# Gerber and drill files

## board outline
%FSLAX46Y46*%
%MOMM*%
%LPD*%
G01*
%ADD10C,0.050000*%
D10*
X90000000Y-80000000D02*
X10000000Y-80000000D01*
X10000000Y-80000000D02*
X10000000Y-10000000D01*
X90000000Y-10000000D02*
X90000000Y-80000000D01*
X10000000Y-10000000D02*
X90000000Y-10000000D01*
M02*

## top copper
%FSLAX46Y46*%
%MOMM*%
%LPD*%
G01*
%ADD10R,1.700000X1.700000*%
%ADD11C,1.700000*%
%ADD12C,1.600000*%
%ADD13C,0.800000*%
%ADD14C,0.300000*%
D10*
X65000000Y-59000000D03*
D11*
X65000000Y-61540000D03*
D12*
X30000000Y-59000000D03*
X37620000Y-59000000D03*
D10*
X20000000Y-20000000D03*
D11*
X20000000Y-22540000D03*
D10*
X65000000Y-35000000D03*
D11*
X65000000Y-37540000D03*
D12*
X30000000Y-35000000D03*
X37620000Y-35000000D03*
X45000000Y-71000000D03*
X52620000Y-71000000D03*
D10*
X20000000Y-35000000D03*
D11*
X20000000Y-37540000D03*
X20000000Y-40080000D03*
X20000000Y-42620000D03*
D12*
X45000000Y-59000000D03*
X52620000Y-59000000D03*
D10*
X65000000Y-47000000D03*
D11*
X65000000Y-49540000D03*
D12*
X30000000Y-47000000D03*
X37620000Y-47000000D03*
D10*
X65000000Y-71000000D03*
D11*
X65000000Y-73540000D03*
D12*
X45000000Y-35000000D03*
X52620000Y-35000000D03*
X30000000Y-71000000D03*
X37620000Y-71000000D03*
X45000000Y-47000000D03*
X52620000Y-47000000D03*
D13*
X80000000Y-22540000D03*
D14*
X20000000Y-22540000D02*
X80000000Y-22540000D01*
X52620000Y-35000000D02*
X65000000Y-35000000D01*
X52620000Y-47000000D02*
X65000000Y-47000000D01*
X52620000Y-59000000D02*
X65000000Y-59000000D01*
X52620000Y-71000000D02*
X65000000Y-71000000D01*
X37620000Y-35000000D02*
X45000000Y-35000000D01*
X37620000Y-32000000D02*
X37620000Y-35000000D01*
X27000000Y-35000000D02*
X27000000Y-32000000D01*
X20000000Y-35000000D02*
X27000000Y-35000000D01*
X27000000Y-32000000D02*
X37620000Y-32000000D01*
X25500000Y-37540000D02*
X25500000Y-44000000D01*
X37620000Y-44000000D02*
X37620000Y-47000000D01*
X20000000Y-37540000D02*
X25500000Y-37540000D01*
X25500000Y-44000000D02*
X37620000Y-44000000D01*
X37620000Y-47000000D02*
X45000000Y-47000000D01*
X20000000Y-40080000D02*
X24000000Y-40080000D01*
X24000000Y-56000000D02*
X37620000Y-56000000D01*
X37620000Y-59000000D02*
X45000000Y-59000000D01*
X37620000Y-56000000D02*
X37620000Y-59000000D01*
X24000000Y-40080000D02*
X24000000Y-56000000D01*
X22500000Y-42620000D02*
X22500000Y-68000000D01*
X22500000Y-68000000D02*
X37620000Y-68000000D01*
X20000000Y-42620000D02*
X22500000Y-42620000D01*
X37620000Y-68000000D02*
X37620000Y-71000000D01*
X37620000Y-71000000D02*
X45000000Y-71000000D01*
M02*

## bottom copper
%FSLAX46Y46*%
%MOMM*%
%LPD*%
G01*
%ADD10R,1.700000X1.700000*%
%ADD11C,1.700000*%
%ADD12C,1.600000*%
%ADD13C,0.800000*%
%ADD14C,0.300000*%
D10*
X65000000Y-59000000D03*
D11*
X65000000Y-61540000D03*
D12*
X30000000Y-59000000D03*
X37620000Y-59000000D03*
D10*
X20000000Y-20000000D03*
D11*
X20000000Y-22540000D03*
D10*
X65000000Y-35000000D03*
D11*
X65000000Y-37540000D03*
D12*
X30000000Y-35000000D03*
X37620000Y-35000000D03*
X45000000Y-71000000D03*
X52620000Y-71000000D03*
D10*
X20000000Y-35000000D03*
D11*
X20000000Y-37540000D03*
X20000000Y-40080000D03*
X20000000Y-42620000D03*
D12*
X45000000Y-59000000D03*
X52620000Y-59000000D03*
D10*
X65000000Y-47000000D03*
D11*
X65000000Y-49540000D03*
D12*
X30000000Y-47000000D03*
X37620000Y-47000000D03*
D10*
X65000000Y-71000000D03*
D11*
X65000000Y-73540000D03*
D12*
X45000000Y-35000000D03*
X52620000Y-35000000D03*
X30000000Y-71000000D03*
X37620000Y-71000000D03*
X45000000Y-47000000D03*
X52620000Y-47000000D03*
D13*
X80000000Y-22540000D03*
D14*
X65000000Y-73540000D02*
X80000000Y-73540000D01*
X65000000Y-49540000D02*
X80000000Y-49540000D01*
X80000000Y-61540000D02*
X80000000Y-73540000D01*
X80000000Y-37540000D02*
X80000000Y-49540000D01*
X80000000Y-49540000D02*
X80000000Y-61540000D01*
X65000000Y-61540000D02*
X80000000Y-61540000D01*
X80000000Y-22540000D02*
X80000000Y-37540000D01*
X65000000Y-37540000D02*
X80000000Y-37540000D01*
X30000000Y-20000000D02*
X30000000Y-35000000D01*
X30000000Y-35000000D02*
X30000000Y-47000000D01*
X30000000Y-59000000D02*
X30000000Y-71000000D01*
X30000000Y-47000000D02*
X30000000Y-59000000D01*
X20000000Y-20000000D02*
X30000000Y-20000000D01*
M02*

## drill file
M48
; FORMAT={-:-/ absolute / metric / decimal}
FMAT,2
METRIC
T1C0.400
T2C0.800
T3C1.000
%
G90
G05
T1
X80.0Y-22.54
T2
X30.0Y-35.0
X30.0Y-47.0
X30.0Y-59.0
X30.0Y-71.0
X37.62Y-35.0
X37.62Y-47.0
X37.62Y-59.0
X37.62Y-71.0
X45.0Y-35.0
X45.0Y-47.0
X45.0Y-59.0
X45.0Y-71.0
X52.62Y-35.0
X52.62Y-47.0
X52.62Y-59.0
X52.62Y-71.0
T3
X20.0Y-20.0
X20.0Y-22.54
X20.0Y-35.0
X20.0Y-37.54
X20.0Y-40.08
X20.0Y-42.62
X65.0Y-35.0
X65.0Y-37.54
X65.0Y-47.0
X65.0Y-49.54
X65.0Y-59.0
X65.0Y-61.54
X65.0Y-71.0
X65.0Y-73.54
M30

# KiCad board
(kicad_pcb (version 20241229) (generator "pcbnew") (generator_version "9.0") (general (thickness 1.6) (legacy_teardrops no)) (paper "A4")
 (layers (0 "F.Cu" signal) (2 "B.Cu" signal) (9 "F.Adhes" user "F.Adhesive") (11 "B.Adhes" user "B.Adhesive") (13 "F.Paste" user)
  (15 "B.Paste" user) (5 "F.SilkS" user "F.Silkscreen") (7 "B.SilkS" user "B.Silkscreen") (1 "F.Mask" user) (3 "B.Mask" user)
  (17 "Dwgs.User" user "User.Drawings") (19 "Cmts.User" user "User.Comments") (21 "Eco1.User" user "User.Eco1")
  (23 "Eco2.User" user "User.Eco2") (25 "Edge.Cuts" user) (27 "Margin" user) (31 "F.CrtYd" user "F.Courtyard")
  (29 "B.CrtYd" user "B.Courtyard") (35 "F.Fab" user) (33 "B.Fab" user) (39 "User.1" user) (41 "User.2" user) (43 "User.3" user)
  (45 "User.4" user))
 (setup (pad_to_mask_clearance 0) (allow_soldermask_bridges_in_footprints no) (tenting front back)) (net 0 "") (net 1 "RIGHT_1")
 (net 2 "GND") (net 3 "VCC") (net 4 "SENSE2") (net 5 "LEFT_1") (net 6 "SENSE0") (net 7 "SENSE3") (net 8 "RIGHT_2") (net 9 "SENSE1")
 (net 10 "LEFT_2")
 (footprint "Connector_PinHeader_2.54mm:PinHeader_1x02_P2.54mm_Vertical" (layer "F.Cu") (at 65 59)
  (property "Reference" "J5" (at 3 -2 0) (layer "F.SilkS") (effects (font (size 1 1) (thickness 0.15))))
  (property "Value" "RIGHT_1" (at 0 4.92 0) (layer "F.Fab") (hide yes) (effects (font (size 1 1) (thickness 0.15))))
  (pad "1" thru_hole rect (at 0 0) (size 1.7 1.7) (drill 1) (layers "*.Cu" "*.Mask") (remove_unused_layers no) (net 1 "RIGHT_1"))
  (pad "2" thru_hole circle (at 0 2.54) (size 1.7 1.7) (drill 1) (layers "*.Cu" "*.Mask") (remove_unused_layers no) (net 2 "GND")))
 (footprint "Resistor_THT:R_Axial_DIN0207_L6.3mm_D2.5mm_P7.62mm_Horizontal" (layer "F.Cu") (at 30 59)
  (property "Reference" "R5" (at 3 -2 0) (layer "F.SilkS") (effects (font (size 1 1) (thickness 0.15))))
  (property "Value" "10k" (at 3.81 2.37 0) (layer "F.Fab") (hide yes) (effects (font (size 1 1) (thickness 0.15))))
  (pad "1" thru_hole circle (at 0 0) (size 1.6 1.6) (drill 0.8) (layers "*.Cu" "*.Mask") (remove_unused_layers no) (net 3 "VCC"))
  (pad "2" thru_hole circle (at 7.62 0) (size 1.6 1.6) (drill 0.8) (layers "*.Cu" "*.Mask") (remove_unused_layers no) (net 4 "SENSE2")))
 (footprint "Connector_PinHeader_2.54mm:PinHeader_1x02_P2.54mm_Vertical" (layer "F.Cu") (at 20 20)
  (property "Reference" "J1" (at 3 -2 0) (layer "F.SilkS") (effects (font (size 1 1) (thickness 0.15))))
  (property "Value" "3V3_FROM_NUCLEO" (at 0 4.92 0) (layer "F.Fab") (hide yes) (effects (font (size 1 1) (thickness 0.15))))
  (pad "1" thru_hole rect (at 0 0) (size 1.7 1.7) (drill 1) (layers "*.Cu" "*.Mask") (remove_unused_layers no) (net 3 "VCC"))
  (pad "2" thru_hole circle (at 0 2.54) (size 1.7 1.7) (drill 1) (layers "*.Cu" "*.Mask") (remove_unused_layers no) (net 2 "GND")))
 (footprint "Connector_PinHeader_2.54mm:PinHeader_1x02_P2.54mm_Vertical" (layer "F.Cu") (at 65 35)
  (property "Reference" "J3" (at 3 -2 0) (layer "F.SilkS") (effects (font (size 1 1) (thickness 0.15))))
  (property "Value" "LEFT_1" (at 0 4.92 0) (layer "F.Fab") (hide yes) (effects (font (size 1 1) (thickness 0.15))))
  (pad "1" thru_hole rect (at 0 0) (size 1.7 1.7) (drill 1) (layers "*.Cu" "*.Mask") (remove_unused_layers no) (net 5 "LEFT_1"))
  (pad "2" thru_hole circle (at 0 2.54) (size 1.7 1.7) (drill 1) (layers "*.Cu" "*.Mask") (remove_unused_layers no) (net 2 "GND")))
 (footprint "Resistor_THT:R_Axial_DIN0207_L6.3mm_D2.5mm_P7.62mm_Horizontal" (layer "F.Cu") (at 30 35)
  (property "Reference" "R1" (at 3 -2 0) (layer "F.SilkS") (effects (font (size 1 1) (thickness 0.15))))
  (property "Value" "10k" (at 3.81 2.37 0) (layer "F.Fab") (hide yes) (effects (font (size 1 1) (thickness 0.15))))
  (pad "1" thru_hole circle (at 0 0) (size 1.6 1.6) (drill 0.8) (layers "*.Cu" "*.Mask") (remove_unused_layers no) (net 3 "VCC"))
  (pad "2" thru_hole circle (at 7.62 0) (size 1.6 1.6) (drill 0.8) (layers "*.Cu" "*.Mask") (remove_unused_layers no) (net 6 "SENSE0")))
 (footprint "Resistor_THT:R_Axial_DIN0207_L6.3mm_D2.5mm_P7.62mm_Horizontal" (layer "F.Cu") (at 45 71)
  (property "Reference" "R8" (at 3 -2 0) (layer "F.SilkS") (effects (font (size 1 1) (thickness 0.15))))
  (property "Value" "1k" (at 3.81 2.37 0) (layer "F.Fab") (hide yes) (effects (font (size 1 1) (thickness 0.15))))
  (pad "1" thru_hole circle (at 0 0) (size 1.6 1.6) (drill 0.8) (layers "*.Cu" "*.Mask") (remove_unused_layers no) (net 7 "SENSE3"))
  (pad "2" thru_hole circle (at 7.62 0) (size 1.6 1.6) (drill 0.8) (layers "*.Cu" "*.Mask") (remove_unused_layers no) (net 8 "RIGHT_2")))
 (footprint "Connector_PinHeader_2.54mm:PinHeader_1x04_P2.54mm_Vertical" (layer "F.Cu") (at 20 35)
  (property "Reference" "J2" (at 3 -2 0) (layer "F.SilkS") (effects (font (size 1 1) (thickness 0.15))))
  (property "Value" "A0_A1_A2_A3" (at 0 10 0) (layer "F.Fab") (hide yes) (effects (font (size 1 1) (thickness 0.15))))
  (pad "1" thru_hole rect (at 0 0) (size 1.7 1.7) (drill 1) (layers "*.Cu" "*.Mask") (remove_unused_layers no) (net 6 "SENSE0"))
  (pad "2" thru_hole circle (at 0 2.54) (size 1.7 1.7) (drill 1) (layers "*.Cu" "*.Mask") (remove_unused_layers no) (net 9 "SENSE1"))
  (pad "3" thru_hole circle (at 0 5.08) (size 1.7 1.7) (drill 1) (layers "*.Cu" "*.Mask") (remove_unused_layers no) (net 4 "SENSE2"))
  (pad "4" thru_hole circle (at 0 7.62) (size 1.7 1.7) (drill 1) (layers "*.Cu" "*.Mask") (remove_unused_layers no) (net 7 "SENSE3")))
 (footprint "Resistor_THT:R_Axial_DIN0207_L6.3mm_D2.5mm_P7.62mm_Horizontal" (layer "F.Cu") (at 45 59)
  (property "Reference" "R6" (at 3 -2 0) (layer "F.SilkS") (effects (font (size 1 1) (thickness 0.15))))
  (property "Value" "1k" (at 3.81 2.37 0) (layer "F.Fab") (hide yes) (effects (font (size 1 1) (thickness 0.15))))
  (pad "1" thru_hole circle (at 0 0) (size 1.6 1.6) (drill 0.8) (layers "*.Cu" "*.Mask") (remove_unused_layers no) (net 4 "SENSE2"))
  (pad "2" thru_hole circle (at 7.62 0) (size 1.6 1.6) (drill 0.8) (layers "*.Cu" "*.Mask") (remove_unused_layers no) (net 1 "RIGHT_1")))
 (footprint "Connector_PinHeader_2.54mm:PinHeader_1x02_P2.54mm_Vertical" (layer "F.Cu") (at 65 47)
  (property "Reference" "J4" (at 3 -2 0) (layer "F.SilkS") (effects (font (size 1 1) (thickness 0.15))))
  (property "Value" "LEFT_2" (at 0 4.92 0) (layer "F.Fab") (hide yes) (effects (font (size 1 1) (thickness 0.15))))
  (pad "1" thru_hole rect (at 0 0) (size 1.7 1.7) (drill 1) (layers "*.Cu" "*.Mask") (remove_unused_layers no) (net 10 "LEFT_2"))
  (pad "2" thru_hole circle (at 0 2.54) (size 1.7 1.7) (drill 1) (layers "*.Cu" "*.Mask") (remove_unused_layers no) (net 2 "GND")))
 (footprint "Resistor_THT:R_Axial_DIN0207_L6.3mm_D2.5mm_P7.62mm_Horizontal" (layer "F.Cu") (at 30 47)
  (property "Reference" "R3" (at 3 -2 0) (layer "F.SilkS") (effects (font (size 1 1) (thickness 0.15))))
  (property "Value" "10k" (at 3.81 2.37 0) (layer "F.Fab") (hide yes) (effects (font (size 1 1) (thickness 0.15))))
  (pad "1" thru_hole circle (at 0 0) (size 1.6 1.6) (drill 0.8) (layers "*.Cu" "*.Mask") (remove_unused_layers no) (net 3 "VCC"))
  (pad "2" thru_hole circle (at 7.62 0) (size 1.6 1.6) (drill 0.8) (layers "*.Cu" "*.Mask") (remove_unused_layers no) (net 9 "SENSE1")))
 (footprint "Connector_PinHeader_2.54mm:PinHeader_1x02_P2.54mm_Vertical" (layer "F.Cu") (at 65 71)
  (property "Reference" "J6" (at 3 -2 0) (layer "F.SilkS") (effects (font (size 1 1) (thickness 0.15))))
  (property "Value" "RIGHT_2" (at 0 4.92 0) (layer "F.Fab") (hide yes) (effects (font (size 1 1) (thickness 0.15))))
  (pad "1" thru_hole rect (at 0 0) (size 1.7 1.7) (drill 1) (layers "*.Cu" "*.Mask") (remove_unused_layers no) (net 8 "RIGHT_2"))
  (pad "2" thru_hole circle (at 0 2.54) (size 1.7 1.7) (drill 1) (layers "*.Cu" "*.Mask") (remove_unused_layers no) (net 2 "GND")))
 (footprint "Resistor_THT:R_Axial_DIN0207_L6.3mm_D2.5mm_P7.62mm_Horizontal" (layer "F.Cu") (at 45 35)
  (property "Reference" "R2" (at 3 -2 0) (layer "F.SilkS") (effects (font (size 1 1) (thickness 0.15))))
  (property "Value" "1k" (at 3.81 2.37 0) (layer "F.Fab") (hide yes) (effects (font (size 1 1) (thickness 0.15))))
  (pad "1" thru_hole circle (at 0 0) (size 1.6 1.6) (drill 0.8) (layers "*.Cu" "*.Mask") (remove_unused_layers no) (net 6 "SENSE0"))
  (pad "2" thru_hole circle (at 7.62 0) (size 1.6 1.6) (drill 0.8) (layers "*.Cu" "*.Mask") (remove_unused_layers no) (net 5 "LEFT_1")))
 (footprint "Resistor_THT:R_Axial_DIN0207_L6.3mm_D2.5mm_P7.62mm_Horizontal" (layer "F.Cu") (at 30 71)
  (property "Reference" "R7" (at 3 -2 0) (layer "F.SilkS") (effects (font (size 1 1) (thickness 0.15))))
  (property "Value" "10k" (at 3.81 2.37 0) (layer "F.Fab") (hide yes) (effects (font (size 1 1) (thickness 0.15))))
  (pad "1" thru_hole circle (at 0 0) (size 1.6 1.6) (drill 0.8) (layers "*.Cu" "*.Mask") (remove_unused_layers no) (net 3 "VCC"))
  (pad "2" thru_hole circle (at 7.62 0) (size 1.6 1.6) (drill 0.8) (layers "*.Cu" "*.Mask") (remove_unused_layers no) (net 7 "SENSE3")))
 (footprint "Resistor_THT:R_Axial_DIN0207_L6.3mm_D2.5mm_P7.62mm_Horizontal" (layer "F.Cu") (at 45 47)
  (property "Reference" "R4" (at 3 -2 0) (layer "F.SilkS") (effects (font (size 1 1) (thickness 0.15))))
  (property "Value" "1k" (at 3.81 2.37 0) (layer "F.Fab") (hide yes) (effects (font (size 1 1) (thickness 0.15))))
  (pad "1" thru_hole circle (at 0 0) (size 1.6 1.6) (drill 0.8) (layers "*.Cu" "*.Mask") (remove_unused_layers no) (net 9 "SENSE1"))
  (pad "2" thru_hole circle (at 7.62 0) (size 1.6 1.6) (drill 0.8) (layers "*.Cu" "*.Mask") (remove_unused_layers no) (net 10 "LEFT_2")))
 (gr_line (start 90 80) (end 10 80) (stroke (width 0.05) (type default)) (layer "Edge.Cuts"))
 (gr_line (start 10 80) (end 10 10) (stroke (width 0.05) (type default)) (layer "Edge.Cuts"))
 (gr_line (start 90 10) (end 90 80) (stroke (width 0.05) (type default)) (layer "Edge.Cuts"))
 (gr_line (start 10 10) (end 90 10) (stroke (width 0.05) (type default)) (layer "Edge.Cuts"))
 (segment (start 20 22.54) (end 80 22.54) (width 0.3) (layer "F.Cu") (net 2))
 (via (at 80 22.54) (size 0.8) (drill 0.4) (layers "F.Cu" "B.Cu") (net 2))
 (segment (start 65 73.54) (end 80 73.54) (width 0.3) (layer "B.Cu") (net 2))
 (segment (start 65 49.54) (end 80 49.54) (width 0.3) (layer "B.Cu") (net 2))
 (segment (start 80 61.54) (end 80 73.54) (width 0.3) (layer "B.Cu") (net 2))
 (segment (start 80 37.54) (end 80 49.54) (width 0.3) (layer "B.Cu") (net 2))
 (segment (start 80 49.54) (end 80 61.54) (width 0.3) (layer "B.Cu") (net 2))
 (segment (start 65 61.54) (end 80 61.54) (width 0.3) (layer "B.Cu") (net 2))
 (segment (start 80 22.54) (end 80 37.54) (width 0.3) (layer "B.Cu") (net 2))
 (segment (start 65 37.54) (end 80 37.54) (width 0.3) (layer "B.Cu") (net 2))
 (segment (start 52.62 35) (end 65 35) (width 0.3) (layer "F.Cu") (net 5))
 (segment (start 52.62 47) (end 65 47) (width 0.3) (layer "F.Cu") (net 10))
 (segment (start 52.62 59) (end 65 59) (width 0.3) (layer "F.Cu") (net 1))
 (segment (start 52.62 71) (end 65 71) (width 0.3) (layer "F.Cu") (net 8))
 (segment (start 37.62 35) (end 45 35) (width 0.3) (layer "F.Cu") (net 6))
 (segment (start 37.62 32) (end 37.62 35) (width 0.3) (layer "F.Cu") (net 6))
 (segment (start 27 35) (end 27 32) (width 0.3) (layer "F.Cu") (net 6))
 (segment (start 20 35) (end 27 35) (width 0.3) (layer "F.Cu") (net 6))
 (segment (start 27 32) (end 37.62 32) (width 0.3) (layer "F.Cu") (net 6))
 (segment (start 25.5 37.54) (end 25.5 44) (width 0.3) (layer "F.Cu") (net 9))
 (segment (start 37.62 44) (end 37.62 47) (width 0.3) (layer "F.Cu") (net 9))
 (segment (start 20 37.54) (end 25.5 37.54) (width 0.3) (layer "F.Cu") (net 9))
 (segment (start 25.5 44) (end 37.62 44) (width 0.3) (layer "F.Cu") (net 9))
 (segment (start 37.62 47) (end 45 47) (width 0.3) (layer "F.Cu") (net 9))
 (segment (start 20 40.08) (end 24 40.08) (width 0.3) (layer "F.Cu") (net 4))
 (segment (start 24 56) (end 37.62 56) (width 0.3) (layer "F.Cu") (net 4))
 (segment (start 37.62 59) (end 45 59) (width 0.3) (layer "F.Cu") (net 4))
 (segment (start 37.62 56) (end 37.62 59) (width 0.3) (layer "F.Cu") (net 4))
 (segment (start 24 40.08) (end 24 56) (width 0.3) (layer "F.Cu") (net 4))
 (segment (start 22.5 42.62) (end 22.5 68) (width 0.3) (layer "F.Cu") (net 7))
 (segment (start 22.5 68) (end 37.62 68) (width 0.3) (layer "F.Cu") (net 7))
 (segment (start 20 42.62) (end 22.5 42.62) (width 0.3) (layer "F.Cu") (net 7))
 (segment (start 37.62 68) (end 37.62 71) (width 0.3) (layer "F.Cu") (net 7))
 (segment (start 37.62 71) (end 45 71) (width 0.3) (layer "F.Cu") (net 7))
 (segment (start 30 20) (end 30 35) (width 0.3) (layer "B.Cu") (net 3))
 (segment (start 30 35) (end 30 47) (width 0.3) (layer "B.Cu") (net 3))
 (segment (start 30 59) (end 30 71) (width 0.3) (layer "B.Cu") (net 3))
 (segment (start 30 47) (end 30 59) (width 0.3) (layer "B.Cu") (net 3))
 (segment (start 20 20) (end 30 20) (width 0.3) (layer "B.Cu") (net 3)))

